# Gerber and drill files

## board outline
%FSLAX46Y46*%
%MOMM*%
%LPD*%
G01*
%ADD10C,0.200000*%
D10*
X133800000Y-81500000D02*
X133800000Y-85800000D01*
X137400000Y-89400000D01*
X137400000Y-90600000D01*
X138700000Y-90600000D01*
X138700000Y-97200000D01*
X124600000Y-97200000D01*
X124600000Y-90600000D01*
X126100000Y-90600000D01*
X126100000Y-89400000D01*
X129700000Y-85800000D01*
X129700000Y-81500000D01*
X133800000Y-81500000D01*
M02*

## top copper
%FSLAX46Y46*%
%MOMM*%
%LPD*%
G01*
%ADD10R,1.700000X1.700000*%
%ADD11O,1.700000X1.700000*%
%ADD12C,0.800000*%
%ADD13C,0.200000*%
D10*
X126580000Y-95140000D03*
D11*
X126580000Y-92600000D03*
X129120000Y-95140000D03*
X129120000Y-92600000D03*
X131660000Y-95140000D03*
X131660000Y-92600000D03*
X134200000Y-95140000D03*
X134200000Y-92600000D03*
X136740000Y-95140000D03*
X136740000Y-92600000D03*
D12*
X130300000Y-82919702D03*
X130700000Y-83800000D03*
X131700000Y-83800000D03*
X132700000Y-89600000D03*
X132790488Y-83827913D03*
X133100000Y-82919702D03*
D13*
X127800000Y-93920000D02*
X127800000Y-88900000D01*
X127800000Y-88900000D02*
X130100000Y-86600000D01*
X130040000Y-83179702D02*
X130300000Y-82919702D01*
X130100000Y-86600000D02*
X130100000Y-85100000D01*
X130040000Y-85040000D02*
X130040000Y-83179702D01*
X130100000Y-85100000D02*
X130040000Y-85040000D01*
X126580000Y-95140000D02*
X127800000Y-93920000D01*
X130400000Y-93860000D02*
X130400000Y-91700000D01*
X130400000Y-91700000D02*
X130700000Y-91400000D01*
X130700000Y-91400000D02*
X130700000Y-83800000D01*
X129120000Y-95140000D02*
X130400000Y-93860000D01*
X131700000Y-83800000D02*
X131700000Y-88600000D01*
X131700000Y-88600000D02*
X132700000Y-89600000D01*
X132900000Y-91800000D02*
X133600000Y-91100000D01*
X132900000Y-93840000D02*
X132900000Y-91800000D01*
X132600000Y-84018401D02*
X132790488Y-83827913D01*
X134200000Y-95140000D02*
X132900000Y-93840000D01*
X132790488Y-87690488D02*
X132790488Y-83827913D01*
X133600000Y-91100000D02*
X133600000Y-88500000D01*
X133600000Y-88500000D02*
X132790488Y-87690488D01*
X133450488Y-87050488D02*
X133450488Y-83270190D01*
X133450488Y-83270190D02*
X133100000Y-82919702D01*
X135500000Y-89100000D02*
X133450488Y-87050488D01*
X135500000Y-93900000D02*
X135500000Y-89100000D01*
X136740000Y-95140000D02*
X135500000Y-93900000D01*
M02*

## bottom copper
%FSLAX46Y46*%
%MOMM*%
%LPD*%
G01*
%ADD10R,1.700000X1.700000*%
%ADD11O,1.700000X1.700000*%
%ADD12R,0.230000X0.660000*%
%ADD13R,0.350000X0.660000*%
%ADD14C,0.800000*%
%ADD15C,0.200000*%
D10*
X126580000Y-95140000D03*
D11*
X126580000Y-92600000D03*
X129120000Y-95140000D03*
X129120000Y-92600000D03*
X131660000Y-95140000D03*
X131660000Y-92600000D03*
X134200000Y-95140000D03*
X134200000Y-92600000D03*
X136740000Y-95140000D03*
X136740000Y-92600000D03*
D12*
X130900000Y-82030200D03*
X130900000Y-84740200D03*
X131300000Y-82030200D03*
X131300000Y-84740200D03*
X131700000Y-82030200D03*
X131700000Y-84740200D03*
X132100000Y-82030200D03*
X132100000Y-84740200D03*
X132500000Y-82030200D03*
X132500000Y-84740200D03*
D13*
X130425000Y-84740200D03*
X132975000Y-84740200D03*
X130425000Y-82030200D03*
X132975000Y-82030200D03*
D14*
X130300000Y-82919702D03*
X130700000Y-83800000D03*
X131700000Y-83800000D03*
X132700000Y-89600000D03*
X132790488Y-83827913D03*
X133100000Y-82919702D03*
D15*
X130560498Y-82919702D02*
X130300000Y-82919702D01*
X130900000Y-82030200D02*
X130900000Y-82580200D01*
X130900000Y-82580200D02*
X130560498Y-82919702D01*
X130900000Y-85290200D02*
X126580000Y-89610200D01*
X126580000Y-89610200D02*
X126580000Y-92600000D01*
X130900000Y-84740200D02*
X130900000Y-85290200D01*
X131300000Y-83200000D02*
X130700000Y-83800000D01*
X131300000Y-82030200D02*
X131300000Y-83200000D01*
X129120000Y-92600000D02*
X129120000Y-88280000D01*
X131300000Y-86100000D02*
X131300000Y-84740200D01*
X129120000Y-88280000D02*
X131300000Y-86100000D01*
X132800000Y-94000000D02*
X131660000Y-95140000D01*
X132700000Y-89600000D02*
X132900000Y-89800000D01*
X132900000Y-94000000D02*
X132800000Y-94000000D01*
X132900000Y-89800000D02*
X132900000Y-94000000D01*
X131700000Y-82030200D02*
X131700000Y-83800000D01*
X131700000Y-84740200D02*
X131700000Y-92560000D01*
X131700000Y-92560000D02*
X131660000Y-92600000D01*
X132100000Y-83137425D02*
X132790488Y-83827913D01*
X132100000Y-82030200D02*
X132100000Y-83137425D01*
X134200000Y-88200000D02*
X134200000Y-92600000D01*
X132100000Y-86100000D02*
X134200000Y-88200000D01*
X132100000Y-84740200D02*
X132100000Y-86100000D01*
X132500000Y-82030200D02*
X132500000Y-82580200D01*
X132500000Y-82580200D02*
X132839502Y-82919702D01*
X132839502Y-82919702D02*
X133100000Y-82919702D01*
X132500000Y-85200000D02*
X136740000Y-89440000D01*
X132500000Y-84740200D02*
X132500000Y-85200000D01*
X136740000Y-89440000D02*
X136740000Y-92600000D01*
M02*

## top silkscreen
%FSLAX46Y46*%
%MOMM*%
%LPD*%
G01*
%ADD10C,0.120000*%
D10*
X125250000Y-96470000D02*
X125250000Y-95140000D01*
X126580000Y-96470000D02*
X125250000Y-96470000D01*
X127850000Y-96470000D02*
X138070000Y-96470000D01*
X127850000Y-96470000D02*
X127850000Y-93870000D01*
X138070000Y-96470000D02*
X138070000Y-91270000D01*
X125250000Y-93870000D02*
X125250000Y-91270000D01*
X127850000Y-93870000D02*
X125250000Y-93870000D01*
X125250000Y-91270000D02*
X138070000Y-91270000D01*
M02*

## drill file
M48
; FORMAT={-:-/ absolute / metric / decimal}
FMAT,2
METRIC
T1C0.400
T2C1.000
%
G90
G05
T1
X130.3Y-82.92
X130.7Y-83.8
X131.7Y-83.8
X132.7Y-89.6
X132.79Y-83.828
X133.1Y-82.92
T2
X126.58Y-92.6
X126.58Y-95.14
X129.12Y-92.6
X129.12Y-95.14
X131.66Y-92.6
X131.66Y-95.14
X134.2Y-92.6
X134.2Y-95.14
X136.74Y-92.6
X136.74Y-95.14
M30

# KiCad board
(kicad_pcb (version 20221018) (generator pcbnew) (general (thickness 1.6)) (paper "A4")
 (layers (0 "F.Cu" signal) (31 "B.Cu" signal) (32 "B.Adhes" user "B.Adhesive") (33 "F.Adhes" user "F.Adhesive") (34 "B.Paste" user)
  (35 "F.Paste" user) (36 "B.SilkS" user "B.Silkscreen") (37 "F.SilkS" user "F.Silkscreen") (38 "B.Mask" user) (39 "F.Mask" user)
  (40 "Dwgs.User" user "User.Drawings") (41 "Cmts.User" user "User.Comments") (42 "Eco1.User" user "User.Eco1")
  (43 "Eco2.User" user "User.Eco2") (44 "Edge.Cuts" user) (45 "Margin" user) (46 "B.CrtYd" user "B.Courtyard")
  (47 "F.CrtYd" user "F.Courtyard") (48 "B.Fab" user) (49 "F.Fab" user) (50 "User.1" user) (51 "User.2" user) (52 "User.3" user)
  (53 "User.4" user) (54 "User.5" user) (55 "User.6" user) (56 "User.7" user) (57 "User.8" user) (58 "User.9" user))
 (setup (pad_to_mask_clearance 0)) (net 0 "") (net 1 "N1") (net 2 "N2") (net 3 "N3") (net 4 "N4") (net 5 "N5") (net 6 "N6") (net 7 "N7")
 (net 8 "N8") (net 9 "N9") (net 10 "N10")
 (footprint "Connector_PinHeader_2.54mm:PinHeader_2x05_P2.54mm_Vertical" (layer "F.Cu") (at 126.58 95.14 90)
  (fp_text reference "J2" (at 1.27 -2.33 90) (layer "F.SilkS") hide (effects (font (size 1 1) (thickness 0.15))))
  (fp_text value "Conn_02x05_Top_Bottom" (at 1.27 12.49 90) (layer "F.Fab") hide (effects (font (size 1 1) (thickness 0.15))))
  (fp_line (start -1.33 -1.33) (end 0 -1.33) (stroke (width 0.12) (type solid)) (layer "F.SilkS"))
  (fp_line (start -1.33 0) (end -1.33 -1.33) (stroke (width 0.12) (type solid)) (layer "F.SilkS"))
  (fp_line (start -1.33 1.27) (end -1.33 11.49) (stroke (width 0.12) (type solid)) (layer "F.SilkS"))
  (fp_line (start -1.33 1.27) (end 1.27 1.27) (stroke (width 0.12) (type solid)) (layer "F.SilkS"))
  (fp_line (start -1.33 11.49) (end 3.87 11.49) (stroke (width 0.12) (type solid)) (layer "F.SilkS"))
  (fp_line (start 1.27 -1.33) (end 3.87 -1.33) (stroke (width 0.12) (type solid)) (layer "F.SilkS"))
  (fp_line (start 1.27 1.27) (end 1.27 -1.33) (stroke (width 0.12) (type solid)) (layer "F.SilkS"))
  (fp_line (start 3.87 -1.33) (end 3.87 11.49) (stroke (width 0.12) (type solid)) (layer "F.SilkS"))
  (pad "1" thru_hole rect (at 0 0 90) (size 1.7 1.7) (drill 1) (layers "*.Cu" "*.Mask") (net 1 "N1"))
  (pad "2" thru_hole oval (at 2.54 0 90) (size 1.7 1.7) (drill 1) (layers "*.Cu" "*.Mask") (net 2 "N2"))
  (pad "3" thru_hole oval (at 0 2.54 90) (size 1.7 1.7) (drill 1) (layers "*.Cu" "*.Mask") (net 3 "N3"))
  (pad "4" thru_hole oval (at 2.54 2.54 90) (size 1.7 1.7) (drill 1) (layers "*.Cu" "*.Mask") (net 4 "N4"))
  (pad "5" thru_hole oval (at 0 5.08 90) (size 1.7 1.7) (drill 1) (layers "*.Cu" "*.Mask") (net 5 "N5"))
  (pad "6" thru_hole oval (at 2.54 5.08 90) (size 1.7 1.7) (drill 1) (layers "*.Cu" "*.Mask") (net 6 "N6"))
  (pad "7" thru_hole oval (at 0 7.62 90) (size 1.7 1.7) (drill 1) (layers "*.Cu" "*.Mask") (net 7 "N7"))
  (pad "8" thru_hole oval (at 2.54 7.62 90) (size 1.7 1.7) (drill 1) (layers "*.Cu" "*.Mask") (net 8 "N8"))
  (pad "9" thru_hole oval (at 0 10.16 90) (size 1.7 1.7) (drill 1) (layers "*.Cu" "*.Mask") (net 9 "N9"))
  (pad "10" thru_hole oval (at 2.54 10.16 90) (size 1.7 1.7) (drill 1) (layers "*.Cu" "*.Mask") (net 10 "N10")))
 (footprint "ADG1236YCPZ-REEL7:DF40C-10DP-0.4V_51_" (layer "B.Cu") (at 131.7 84.7402)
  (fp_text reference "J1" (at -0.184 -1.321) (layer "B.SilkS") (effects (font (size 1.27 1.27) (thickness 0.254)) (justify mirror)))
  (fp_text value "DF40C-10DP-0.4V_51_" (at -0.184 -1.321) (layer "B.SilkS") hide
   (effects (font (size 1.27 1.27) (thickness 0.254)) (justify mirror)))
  (pad "1" smd rect (at -0.8 -2.71) (size 0.23 0.66) (layers "B.Cu" "B.Paste" "B.Mask") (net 1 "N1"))
  (pad "2" smd rect (at -0.8 0) (size 0.23 0.66) (layers "B.Cu" "B.Paste" "B.Mask") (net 2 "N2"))
  (pad "3" smd rect (at -0.4 -2.71) (size 0.23 0.66) (layers "B.Cu" "B.Paste" "B.Mask") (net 3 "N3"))
  (pad "4" smd rect (at -0.4 0) (size 0.23 0.66) (layers "B.Cu" "B.Paste" "B.Mask") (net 4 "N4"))
  (pad "5" smd rect (at 0 -2.71) (size 0.23 0.66) (layers "B.Cu" "B.Paste" "B.Mask") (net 5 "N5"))
  (pad "6" smd rect (at 0 0) (size 0.23 0.66) (layers "B.Cu" "B.Paste" "B.Mask") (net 6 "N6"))
  (pad "7" smd rect (at 0.4 -2.71) (size 0.23 0.66) (layers "B.Cu" "B.Paste" "B.Mask") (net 7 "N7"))
  (pad "8" smd rect (at 0.4 0) (size 0.23 0.66) (layers "B.Cu" "B.Paste" "B.Mask") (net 8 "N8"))
  (pad "9" smd rect (at 0.8 -2.71) (size 0.23 0.66) (layers "B.Cu" "B.Paste" "B.Mask") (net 9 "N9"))
  (pad "10" smd rect (at 0.8 0) (size 0.23 0.66) (layers "B.Cu" "B.Paste" "B.Mask") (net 10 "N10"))
  (pad "11" smd rect (at -1.275 0) (size 0.35 0.66) (layers "B.Cu" "B.Paste" "B.Mask"))
  (pad "12" smd rect (at 1.275 0) (size 0.35 0.66) (layers "B.Cu" "B.Paste" "B.Mask"))
  (pad "13" smd rect (at -1.275 -2.71) (size 0.35 0.66) (layers "B.Cu" "B.Paste" "B.Mask"))
  (pad "14" smd rect (at 1.275 -2.71) (size 0.35 0.66) (layers "B.Cu" "B.Paste" "B.Mask")))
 (gr_poly
  (pts (xy 133.8 81.5) (xy 133.8 85.8) (xy 137.4 89.4) (xy 137.4 90.6) (xy 138.7 90.6) (xy 138.7 97.2) (xy 124.6 97.2) (xy 124.6 90.6)
   (xy 126.1 90.6) (xy 126.1 89.4) (xy 129.7 85.8) (xy 129.7 81.5))
  (stroke (width 0.2) (type solid)) (fill none) (layer "Edge.Cuts"))
 (segment (start 127.8 93.92) (end 127.8 88.9) (width 0.2) (layer "F.Cu") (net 1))
 (segment (start 127.8 88.9) (end 130.1 86.6) (width 0.2) (layer "F.Cu") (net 1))
 (segment (start 130.04 83.179702) (end 130.3 82.919702) (width 0.2) (layer "F.Cu") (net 1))
 (segment (start 130.1 86.6) (end 130.1 85.1) (width 0.2) (layer "F.Cu") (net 1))
 (segment (start 130.04 85.04) (end 130.04 83.179702) (width 0.2) (layer "F.Cu") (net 1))
 (segment (start 130.1 85.1) (end 130.04 85.04) (width 0.2) (layer "F.Cu") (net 1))
 (segment (start 126.58 95.14) (end 127.8 93.92) (width 0.2) (layer "F.Cu") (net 1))
 (via (at 130.3 82.919702) (size 0.8) (drill 0.4) (layers "F.Cu" "B.Cu") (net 1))
 (segment (start 130.560498 82.919702) (end 130.3 82.919702) (width 0.2) (layer "B.Cu") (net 1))
 (segment (start 130.9 82.0302) (end 130.9 82.5802) (width 0.2) (layer "B.Cu") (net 1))
 (segment (start 130.9 82.5802) (end 130.560498 82.919702) (width 0.2) (layer "B.Cu") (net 1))
 (segment (start 130.9 85.2902) (end 126.58 89.6102) (width 0.2) (layer "B.Cu") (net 2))
 (segment (start 126.58 89.6102) (end 126.58 92.6) (width 0.2) (layer "B.Cu") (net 2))
 (segment (start 130.9 84.7402) (end 130.9 85.2902) (width 0.2) (layer "B.Cu") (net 2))
 (segment (start 130.4 93.86) (end 130.4 91.7) (width 0.2) (layer "F.Cu") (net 3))
 (segment (start 130.4 91.7) (end 130.7 91.4) (width 0.2) (layer "F.Cu") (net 3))
 (segment (start 130.7 91.4) (end 130.7 83.8) (width 0.2) (layer "F.Cu") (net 3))
 (segment (start 129.12 95.14) (end 130.4 93.86) (width 0.2) (layer "F.Cu") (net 3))
 (via (at 130.7 83.8) (size 0.8) (drill 0.4) (layers "F.Cu" "B.Cu") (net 3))
 (segment (start 131.3 83.2) (end 130.7 83.8) (width 0.2) (layer "B.Cu") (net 3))
 (segment (start 131.3 82.0302) (end 131.3 83.2) (width 0.2) (layer "B.Cu") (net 3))
 (segment (start 129.12 92.6) (end 129.12 88.28) (width 0.2) (layer "B.Cu") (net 4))
 (segment (start 131.3 86.1) (end 131.3 84.7402) (width 0.2) (layer "B.Cu") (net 4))
 (segment (start 129.12 88.28) (end 131.3 86.1) (width 0.2) (layer "B.Cu") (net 4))
 (segment (start 131.7 83.8) (end 131.7 88.6) (width 0.2) (layer "F.Cu") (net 5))
 (segment (start 131.7 88.6) (end 132.7 89.6) (width 0.2) (layer "F.Cu") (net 5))
 (via (at 131.7 83.8) (size 0.8) (drill 0.4) (layers "F.Cu" "B.Cu") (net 5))
 (via (at 132.7 89.6) (size 0.8) (drill 0.4) (layers "F.Cu" "B.Cu") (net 5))
 (segment (start 132.8 94) (end 131.66 95.14) (width 0.2) (layer "B.Cu") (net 5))
 (segment (start 132.7 89.6) (end 132.9 89.8) (width 0.2) (layer "B.Cu") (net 5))
 (segment (start 132.9 94) (end 132.8 94) (width 0.2) (layer "B.Cu") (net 5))
 (segment (start 132.9 89.8) (end 132.9 94) (width 0.2) (layer "B.Cu") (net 5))
 (segment (start 131.7 82.0302) (end 131.7 83.8) (width 0.2) (layer "B.Cu") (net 5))
 (segment (start 131.7 84.7402) (end 131.7 92.56) (width 0.2) (layer "B.Cu") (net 6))
 (segment (start 131.7 92.56) (end 131.66 92.6) (width 0.2) (layer "B.Cu") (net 6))
 (segment (start 132.9 91.8) (end 133.6 91.1) (width 0.2) (layer "F.Cu") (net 7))
 (segment (start 132.9 93.84) (end 132.9 91.8) (width 0.2) (layer "F.Cu") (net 7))
 (segment (start 132.6 84.018401) (end 132.790488 83.827913) (width 0.2) (layer "F.Cu") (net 7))
 (segment (start 134.2 95.14) (end 132.9 93.84) (width 0.2) (layer "F.Cu") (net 7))
 (segment (start 132.790488 87.690488) (end 132.790488 83.827913) (width 0.2) (layer "F.Cu") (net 7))
 (segment (start 133.6 91.1) (end 133.6 88.5) (width 0.2) (layer "F.Cu") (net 7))
 (segment (start 133.6 88.5) (end 132.790488 87.690488) (width 0.2) (layer "F.Cu") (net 7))
 (via (at 132.790488 83.827913) (size 0.8) (drill 0.4) (layers "F.Cu" "B.Cu") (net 7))
 (segment (start 132.1 83.137425) (end 132.790488 83.827913) (width 0.2) (layer "B.Cu") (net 7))
 (segment (start 132.1 82.0302) (end 132.1 83.137425) (width 0.2) (layer "B.Cu") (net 7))
 (segment (start 134.2 88.2) (end 134.2 92.6) (width 0.2) (layer "B.Cu") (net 8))
 (segment (start 132.1 86.1) (end 134.2 88.2) (width 0.2) (layer "B.Cu") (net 8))
 (segment (start 132.1 84.7402) (end 132.1 86.1) (width 0.2) (layer "B.Cu") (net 8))
 (segment (start 133.450488 87.050488) (end 133.450488 83.27019) (width 0.2) (layer "F.Cu") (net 9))
 (segment (start 133.450488 83.27019) (end 133.1 82.919702) (width 0.2) (layer "F.Cu") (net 9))
 (segment (start 135.5 89.1) (end 133.450488 87.050488) (width 0.2) (layer "F.Cu") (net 9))
 (segment (start 135.5 93.9) (end 135.5 89.1) (width 0.2) (layer "F.Cu") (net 9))
 (segment (start 136.74 95.14) (end 135.5 93.9) (width 0.2) (layer "F.Cu") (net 9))
 (via (at 133.1 82.919702) (size 0.8) (drill 0.4) (layers "F.Cu" "B.Cu") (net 9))
 (segment (start 132.5 82.0302) (end 132.5 82.5802) (width 0.2) (layer "B.Cu") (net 9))
 (segment (start 132.5 82.5802) (end 132.839502 82.919702) (width 0.2) (layer "B.Cu") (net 9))
 (segment (start 132.839502 82.919702) (end 133.1 82.919702) (width 0.2) (layer "B.Cu") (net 9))
 (segment (start 132.5 85.2) (end 136.74 89.44) (width 0.2) (layer "B.Cu") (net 10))
 (segment (start 132.5 84.7402) (end 132.5 85.2) (width 0.2) (layer "B.Cu") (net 10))
 (segment (start 136.74 89.44) (end 136.74 92.6) (width 0.2) (layer "B.Cu") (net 10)))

